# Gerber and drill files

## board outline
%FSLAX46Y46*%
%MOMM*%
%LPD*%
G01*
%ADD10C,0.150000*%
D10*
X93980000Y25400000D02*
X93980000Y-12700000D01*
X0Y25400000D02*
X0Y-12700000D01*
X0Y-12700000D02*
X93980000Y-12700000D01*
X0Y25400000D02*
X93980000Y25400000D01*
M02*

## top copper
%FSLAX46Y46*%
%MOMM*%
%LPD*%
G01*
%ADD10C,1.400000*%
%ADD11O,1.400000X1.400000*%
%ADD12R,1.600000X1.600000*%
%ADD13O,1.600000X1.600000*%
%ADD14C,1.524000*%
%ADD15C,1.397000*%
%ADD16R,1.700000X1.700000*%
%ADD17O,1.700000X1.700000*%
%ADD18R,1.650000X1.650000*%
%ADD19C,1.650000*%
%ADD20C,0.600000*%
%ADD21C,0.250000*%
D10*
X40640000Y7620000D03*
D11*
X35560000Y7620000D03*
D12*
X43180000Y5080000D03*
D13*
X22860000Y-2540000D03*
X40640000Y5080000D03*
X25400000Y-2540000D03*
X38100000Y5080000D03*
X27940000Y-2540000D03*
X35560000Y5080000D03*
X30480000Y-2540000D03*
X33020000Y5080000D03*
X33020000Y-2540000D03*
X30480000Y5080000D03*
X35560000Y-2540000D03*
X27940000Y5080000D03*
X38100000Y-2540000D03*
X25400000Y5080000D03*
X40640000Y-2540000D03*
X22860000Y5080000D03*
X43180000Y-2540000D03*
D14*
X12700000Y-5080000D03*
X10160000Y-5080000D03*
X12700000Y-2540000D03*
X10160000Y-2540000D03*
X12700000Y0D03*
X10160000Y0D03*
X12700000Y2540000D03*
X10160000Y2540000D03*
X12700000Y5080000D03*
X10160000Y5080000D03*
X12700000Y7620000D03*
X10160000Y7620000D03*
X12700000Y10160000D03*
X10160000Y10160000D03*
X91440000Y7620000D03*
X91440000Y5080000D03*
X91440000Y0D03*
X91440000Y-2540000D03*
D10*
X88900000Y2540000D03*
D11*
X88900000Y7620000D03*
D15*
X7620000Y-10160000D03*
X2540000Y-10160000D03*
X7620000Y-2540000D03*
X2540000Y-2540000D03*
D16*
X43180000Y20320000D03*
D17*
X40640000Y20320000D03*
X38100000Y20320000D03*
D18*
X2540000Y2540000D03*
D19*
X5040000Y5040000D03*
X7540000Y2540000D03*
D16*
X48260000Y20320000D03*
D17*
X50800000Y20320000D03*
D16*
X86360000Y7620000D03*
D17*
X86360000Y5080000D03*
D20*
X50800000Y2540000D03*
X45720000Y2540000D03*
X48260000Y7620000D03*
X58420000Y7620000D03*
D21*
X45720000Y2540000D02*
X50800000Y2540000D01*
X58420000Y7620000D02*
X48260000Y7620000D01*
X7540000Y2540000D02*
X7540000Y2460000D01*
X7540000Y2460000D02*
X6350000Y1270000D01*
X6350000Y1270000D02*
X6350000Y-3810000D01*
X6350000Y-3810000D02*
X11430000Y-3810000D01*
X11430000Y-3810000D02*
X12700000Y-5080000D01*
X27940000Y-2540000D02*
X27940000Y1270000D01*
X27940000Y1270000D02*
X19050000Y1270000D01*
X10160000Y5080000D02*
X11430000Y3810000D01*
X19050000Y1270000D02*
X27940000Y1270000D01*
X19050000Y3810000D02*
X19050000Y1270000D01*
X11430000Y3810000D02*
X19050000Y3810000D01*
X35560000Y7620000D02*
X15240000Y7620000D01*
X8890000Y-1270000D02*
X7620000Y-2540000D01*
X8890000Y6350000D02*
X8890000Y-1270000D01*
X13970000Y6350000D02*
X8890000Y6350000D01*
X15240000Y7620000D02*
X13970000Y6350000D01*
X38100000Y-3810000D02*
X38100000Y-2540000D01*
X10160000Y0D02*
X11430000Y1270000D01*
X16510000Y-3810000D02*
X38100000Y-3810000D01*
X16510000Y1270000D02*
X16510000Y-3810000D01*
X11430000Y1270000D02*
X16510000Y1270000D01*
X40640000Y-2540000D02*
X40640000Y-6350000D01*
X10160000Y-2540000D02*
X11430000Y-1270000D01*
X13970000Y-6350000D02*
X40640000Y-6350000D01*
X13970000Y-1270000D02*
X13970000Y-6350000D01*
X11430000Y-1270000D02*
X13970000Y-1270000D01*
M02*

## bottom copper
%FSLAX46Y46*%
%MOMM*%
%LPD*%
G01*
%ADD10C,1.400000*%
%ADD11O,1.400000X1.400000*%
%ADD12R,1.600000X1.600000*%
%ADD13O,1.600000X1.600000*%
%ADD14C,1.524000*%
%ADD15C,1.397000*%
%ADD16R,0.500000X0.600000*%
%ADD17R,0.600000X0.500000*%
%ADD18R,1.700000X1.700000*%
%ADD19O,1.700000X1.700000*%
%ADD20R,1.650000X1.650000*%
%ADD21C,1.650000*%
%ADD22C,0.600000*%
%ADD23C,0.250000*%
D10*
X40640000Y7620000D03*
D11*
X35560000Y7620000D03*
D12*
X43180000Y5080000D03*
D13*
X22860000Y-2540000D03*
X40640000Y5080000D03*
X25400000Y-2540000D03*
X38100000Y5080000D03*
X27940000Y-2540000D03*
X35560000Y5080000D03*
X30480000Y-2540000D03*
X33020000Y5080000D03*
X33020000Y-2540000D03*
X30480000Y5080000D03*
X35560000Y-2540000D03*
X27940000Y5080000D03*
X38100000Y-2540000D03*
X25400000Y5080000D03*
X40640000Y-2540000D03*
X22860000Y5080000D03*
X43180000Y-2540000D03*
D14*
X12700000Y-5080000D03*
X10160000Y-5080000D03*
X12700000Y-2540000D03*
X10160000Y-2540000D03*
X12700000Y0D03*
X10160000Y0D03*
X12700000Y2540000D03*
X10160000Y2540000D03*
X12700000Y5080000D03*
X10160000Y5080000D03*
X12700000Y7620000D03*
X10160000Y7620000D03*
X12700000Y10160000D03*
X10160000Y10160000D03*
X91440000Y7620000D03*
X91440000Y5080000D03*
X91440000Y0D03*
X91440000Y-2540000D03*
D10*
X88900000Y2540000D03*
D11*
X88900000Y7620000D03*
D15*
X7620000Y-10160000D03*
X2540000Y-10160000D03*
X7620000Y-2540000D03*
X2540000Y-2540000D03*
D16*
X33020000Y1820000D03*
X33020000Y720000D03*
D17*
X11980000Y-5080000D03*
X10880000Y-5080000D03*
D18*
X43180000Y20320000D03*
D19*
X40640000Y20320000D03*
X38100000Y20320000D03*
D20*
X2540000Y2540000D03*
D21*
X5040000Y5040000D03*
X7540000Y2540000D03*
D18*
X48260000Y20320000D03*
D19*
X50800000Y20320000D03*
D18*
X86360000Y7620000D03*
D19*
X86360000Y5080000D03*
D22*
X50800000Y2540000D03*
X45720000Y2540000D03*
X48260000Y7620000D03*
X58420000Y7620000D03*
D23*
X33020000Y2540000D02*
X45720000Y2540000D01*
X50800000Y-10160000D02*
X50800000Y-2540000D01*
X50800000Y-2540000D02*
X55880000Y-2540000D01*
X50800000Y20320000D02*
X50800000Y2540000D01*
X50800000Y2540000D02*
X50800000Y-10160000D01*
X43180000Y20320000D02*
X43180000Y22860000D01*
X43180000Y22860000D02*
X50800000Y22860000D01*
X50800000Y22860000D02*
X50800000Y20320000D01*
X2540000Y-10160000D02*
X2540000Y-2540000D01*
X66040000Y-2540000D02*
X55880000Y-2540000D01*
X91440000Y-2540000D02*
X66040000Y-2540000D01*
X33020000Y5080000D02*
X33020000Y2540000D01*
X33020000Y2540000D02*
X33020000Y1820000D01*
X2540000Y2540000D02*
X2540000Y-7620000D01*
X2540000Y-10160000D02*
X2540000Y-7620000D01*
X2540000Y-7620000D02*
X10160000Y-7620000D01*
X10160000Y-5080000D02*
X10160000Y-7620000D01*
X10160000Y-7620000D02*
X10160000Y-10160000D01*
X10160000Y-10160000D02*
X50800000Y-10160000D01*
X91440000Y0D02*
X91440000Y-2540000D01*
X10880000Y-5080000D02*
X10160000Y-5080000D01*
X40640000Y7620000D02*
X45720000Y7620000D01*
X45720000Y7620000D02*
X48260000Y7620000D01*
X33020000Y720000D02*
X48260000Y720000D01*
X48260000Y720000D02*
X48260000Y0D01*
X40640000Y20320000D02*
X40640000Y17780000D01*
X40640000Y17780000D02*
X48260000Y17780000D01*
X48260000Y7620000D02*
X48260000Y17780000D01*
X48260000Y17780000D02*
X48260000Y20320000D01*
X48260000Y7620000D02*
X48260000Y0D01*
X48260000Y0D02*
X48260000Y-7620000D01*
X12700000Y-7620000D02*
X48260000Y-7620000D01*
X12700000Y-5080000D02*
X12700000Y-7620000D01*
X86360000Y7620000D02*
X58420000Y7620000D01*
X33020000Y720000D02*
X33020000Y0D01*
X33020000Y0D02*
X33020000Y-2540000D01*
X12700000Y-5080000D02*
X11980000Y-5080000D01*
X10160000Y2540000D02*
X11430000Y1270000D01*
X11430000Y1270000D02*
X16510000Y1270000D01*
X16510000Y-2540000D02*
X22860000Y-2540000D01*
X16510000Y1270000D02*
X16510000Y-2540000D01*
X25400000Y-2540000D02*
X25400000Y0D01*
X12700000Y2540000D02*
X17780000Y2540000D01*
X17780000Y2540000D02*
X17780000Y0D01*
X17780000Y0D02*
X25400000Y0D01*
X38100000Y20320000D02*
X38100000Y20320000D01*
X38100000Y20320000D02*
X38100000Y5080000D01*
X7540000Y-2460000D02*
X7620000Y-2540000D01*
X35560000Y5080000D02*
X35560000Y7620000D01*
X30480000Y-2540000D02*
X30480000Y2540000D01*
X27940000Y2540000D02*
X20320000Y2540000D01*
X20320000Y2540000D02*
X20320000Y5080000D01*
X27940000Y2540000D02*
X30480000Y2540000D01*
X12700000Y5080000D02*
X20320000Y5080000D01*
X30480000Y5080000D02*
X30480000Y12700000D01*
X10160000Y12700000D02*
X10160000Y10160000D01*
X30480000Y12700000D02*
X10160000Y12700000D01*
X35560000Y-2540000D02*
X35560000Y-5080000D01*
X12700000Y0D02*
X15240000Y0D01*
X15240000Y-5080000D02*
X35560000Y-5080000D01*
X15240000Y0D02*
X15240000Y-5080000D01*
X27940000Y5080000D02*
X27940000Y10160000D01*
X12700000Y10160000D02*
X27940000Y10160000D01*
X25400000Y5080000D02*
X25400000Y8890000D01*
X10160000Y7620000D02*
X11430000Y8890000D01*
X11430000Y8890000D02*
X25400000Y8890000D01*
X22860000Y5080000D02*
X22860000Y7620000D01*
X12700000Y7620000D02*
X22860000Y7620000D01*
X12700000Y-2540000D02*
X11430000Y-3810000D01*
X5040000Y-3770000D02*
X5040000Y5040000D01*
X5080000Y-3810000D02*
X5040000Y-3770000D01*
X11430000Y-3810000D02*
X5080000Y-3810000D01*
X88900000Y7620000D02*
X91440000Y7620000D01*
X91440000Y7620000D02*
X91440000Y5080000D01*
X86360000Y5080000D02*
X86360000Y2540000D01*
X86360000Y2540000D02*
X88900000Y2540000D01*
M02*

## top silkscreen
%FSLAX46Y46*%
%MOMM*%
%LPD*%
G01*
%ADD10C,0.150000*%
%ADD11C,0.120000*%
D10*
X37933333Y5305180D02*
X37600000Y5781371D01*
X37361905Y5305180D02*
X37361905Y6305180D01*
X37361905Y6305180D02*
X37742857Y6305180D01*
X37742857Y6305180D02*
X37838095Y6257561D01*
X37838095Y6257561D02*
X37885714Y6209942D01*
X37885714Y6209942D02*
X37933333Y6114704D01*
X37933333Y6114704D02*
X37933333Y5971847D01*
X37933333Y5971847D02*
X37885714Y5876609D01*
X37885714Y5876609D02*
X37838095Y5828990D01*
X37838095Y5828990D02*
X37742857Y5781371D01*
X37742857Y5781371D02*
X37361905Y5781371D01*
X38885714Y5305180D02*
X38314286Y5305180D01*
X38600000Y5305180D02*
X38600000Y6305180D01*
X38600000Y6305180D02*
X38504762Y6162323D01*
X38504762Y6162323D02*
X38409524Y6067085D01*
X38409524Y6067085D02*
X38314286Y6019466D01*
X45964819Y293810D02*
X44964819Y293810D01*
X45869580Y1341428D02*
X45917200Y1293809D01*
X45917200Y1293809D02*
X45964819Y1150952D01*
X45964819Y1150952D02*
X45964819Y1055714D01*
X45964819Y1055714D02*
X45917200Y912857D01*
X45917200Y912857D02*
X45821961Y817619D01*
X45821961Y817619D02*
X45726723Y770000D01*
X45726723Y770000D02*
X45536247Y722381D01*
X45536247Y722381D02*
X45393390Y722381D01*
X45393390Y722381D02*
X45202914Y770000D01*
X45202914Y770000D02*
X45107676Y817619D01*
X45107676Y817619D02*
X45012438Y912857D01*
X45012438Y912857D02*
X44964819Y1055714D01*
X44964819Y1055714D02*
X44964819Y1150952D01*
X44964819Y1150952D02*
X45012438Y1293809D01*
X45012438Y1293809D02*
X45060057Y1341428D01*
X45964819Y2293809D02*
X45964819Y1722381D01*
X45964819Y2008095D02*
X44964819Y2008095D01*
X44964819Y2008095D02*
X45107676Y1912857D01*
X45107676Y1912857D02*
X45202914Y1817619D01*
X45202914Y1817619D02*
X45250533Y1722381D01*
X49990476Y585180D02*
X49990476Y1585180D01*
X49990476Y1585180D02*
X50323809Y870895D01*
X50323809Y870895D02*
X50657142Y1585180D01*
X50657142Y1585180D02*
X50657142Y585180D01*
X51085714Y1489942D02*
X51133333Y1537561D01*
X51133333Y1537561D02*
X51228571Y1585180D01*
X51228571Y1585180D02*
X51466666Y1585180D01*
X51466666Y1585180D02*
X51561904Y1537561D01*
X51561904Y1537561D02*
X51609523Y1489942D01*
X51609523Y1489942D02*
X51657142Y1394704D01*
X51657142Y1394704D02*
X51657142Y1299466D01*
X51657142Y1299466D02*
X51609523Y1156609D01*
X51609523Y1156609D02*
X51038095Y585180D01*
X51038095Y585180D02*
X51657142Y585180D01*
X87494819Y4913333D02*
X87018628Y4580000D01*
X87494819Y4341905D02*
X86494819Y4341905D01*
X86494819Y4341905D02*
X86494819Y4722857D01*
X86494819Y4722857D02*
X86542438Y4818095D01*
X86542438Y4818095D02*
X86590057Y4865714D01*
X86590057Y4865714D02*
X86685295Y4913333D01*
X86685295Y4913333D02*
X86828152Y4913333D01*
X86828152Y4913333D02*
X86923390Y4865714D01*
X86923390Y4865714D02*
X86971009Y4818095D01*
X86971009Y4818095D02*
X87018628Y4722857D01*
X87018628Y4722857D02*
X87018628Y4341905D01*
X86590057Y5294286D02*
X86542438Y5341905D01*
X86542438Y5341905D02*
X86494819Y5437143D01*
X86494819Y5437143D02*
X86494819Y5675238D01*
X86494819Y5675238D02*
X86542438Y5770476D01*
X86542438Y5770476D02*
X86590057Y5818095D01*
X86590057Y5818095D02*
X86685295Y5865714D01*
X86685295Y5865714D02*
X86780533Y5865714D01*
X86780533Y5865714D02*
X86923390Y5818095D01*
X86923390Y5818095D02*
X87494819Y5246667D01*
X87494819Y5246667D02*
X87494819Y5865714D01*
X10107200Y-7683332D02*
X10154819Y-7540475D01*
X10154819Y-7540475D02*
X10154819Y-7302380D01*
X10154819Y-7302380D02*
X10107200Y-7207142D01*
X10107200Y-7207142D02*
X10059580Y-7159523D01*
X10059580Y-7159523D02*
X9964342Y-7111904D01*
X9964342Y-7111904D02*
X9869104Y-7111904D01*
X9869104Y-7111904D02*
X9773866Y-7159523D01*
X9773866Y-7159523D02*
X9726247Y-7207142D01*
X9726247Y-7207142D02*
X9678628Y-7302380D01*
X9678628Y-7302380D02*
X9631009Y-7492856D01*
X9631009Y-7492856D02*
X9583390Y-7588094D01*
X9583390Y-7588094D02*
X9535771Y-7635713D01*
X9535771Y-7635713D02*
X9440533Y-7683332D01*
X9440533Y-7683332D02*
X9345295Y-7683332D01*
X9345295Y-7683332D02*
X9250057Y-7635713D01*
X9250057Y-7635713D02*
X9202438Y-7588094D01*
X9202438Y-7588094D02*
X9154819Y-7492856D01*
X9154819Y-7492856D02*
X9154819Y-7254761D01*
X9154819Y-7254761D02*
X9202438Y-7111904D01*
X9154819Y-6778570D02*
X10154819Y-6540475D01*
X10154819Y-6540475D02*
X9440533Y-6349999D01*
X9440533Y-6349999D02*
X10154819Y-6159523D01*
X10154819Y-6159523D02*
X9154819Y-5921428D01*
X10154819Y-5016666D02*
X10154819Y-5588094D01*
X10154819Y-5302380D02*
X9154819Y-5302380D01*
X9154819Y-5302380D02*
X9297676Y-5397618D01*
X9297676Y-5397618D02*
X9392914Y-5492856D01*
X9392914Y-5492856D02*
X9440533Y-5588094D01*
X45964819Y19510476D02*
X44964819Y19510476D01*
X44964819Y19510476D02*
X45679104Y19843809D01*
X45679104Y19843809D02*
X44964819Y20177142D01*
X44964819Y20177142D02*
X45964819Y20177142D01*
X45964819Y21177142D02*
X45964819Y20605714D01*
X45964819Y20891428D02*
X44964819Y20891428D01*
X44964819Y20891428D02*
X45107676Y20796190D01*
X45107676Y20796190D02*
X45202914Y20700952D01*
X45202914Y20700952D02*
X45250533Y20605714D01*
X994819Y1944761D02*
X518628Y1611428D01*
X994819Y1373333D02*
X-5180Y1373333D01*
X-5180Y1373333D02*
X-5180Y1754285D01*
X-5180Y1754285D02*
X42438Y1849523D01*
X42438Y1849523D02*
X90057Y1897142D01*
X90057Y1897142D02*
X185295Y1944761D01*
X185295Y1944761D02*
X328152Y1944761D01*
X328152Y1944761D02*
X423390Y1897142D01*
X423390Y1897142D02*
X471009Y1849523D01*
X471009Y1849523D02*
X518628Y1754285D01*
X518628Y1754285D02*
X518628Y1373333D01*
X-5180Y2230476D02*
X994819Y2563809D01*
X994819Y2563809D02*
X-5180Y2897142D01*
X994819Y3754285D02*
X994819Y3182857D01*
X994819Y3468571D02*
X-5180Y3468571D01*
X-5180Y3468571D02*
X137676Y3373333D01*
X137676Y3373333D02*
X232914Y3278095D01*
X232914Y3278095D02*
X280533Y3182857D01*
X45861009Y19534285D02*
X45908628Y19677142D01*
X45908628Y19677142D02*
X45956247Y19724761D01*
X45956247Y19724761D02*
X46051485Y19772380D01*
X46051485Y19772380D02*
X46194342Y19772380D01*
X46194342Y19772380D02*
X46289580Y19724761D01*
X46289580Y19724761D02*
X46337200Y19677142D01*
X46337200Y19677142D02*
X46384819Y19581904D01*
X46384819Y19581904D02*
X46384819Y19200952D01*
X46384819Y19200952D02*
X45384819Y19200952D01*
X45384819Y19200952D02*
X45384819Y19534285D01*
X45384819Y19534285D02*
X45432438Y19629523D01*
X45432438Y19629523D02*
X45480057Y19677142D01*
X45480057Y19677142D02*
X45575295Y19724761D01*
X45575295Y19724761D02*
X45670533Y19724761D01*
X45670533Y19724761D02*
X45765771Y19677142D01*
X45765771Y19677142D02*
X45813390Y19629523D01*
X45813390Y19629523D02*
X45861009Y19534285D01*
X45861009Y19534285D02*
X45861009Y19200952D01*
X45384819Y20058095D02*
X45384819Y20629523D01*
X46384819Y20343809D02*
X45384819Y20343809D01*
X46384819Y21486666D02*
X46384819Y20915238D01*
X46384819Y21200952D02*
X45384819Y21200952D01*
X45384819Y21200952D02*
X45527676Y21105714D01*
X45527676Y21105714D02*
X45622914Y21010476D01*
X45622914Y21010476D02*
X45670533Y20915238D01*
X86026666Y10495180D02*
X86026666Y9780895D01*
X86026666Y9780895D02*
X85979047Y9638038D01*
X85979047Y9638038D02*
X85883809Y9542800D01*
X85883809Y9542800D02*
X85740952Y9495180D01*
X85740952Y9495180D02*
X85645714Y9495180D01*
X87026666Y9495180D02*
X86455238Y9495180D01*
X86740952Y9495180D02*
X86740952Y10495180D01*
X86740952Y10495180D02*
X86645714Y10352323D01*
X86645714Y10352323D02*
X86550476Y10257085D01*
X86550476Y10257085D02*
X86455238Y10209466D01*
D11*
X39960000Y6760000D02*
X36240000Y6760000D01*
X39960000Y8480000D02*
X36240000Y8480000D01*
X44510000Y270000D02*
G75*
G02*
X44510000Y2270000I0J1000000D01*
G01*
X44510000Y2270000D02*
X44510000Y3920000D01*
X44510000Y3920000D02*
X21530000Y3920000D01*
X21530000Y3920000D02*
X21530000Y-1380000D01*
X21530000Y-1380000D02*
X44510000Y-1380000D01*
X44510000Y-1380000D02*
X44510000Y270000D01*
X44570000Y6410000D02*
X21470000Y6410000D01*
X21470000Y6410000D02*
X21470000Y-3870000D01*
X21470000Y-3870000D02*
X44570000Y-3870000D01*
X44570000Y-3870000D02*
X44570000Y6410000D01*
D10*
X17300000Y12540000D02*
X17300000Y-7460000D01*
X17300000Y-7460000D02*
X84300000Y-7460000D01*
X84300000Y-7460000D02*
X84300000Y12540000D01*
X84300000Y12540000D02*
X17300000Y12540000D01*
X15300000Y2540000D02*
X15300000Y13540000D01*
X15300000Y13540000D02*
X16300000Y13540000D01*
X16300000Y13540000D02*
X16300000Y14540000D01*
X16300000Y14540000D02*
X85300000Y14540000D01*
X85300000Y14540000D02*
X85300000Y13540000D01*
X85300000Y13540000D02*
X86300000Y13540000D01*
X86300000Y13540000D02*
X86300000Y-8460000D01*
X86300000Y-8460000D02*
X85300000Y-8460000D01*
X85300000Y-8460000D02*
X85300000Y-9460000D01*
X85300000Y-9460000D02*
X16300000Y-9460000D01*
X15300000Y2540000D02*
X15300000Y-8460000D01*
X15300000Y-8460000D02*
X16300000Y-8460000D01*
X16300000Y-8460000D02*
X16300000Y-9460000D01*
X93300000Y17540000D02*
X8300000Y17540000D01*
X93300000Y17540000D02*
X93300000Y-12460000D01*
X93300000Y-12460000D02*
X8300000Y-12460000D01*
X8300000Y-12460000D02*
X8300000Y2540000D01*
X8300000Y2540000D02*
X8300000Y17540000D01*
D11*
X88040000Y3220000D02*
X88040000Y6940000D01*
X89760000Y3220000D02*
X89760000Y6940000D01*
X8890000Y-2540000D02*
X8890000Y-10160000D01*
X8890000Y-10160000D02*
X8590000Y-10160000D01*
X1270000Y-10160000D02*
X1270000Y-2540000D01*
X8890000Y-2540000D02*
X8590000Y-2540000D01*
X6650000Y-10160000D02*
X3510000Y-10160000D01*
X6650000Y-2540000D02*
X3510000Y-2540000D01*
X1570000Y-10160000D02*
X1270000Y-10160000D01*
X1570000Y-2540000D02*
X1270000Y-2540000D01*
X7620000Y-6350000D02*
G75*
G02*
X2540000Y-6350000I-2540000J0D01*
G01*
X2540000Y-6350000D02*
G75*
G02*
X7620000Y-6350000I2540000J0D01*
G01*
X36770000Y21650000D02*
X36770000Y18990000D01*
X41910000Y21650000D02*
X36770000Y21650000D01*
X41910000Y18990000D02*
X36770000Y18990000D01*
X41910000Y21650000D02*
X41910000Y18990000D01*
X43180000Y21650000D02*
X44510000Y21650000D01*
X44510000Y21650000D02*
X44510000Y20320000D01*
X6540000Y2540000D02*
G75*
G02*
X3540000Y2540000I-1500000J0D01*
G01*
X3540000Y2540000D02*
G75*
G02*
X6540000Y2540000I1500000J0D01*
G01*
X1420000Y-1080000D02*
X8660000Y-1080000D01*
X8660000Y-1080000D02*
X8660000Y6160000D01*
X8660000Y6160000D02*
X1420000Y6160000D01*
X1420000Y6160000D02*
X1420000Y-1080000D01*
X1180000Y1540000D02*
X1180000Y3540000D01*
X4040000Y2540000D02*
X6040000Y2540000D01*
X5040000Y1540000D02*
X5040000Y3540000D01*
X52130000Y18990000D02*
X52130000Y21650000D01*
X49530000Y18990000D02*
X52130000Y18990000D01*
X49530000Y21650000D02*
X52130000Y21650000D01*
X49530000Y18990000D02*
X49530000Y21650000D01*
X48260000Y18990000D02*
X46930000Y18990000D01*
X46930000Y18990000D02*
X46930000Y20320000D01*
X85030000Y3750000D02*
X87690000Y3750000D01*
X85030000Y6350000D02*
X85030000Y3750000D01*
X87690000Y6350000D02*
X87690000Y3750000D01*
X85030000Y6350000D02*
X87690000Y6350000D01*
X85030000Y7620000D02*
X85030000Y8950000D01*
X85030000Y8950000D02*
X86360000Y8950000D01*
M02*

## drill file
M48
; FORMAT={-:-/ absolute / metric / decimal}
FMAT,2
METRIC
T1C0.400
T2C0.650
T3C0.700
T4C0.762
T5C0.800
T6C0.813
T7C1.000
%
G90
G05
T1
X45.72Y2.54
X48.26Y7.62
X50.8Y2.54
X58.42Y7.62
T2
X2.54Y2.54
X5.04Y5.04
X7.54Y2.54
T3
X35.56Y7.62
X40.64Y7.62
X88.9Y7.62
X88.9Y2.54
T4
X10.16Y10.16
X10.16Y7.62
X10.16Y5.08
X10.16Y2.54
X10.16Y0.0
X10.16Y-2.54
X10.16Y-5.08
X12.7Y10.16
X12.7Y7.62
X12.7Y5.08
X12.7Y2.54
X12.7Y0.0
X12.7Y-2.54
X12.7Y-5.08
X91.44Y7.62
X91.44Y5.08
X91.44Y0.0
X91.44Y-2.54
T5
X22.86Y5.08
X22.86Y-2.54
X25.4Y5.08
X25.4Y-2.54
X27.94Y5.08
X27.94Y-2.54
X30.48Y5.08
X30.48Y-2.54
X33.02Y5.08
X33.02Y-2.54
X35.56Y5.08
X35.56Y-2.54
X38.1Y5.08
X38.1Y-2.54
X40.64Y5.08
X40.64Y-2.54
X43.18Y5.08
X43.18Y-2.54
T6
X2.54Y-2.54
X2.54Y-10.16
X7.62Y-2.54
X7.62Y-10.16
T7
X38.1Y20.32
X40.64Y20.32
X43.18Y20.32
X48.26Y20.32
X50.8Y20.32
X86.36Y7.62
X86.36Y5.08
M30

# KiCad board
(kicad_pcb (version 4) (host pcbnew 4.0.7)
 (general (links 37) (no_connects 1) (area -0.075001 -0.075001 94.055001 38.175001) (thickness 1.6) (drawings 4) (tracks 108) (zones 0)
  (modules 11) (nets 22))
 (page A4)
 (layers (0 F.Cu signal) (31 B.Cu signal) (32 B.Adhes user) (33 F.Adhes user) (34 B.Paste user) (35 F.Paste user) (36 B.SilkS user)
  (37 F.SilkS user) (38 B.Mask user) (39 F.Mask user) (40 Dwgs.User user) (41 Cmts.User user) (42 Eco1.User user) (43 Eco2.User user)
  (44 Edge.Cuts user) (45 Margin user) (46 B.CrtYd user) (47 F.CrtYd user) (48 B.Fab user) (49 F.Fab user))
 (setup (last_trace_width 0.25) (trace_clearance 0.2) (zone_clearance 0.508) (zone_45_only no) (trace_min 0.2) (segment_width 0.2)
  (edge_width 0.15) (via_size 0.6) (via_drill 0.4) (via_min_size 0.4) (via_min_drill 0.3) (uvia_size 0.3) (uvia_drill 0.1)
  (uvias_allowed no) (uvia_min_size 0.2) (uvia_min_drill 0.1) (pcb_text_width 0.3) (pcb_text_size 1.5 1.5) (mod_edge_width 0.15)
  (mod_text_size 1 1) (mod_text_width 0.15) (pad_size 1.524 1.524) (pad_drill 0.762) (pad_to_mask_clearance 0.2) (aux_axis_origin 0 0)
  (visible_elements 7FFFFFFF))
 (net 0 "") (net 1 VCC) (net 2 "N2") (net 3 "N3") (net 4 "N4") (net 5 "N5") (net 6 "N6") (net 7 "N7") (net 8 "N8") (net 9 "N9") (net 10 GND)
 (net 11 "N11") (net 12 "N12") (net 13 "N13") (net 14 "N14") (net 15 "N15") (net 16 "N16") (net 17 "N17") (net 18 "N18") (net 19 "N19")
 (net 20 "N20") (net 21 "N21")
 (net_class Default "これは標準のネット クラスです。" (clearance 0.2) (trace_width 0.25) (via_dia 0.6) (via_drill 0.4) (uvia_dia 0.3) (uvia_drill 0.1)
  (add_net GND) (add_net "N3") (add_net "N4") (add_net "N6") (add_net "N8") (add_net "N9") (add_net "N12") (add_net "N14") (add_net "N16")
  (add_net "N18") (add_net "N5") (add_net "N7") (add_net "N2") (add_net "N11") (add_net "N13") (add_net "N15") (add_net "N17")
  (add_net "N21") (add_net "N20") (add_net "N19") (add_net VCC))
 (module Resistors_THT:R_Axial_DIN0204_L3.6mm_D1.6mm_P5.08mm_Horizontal (layer F.Cu) (at 40.64 -7.62 180)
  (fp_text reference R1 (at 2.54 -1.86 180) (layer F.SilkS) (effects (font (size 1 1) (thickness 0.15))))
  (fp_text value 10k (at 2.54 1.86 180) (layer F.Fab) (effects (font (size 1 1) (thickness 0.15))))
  (fp_line (start 0.68 -0.86) (end 4.4 -0.86) (layer F.SilkS) (width 0.12))
  (fp_line (start 0.68 0.86) (end 4.4 0.86) (layer F.SilkS) (width 0.12))
  (pad 1 thru_hole circle (at 0 0 180) (size 1.4 1.4) (drill 0.7) (layers *.Cu *.Mask) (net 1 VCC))
  (pad 2 thru_hole oval (at 5.08 0 180) (size 1.4 1.4) (drill 0.7) (layers *.Cu *.Mask) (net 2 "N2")))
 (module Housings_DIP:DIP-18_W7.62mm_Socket (layer F.Cu) (at 43.18 -5.08 270)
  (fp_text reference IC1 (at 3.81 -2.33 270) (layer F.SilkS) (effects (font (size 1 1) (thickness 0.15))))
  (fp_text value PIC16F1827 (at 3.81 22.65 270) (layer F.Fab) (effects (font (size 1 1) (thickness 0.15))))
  (fp_arc (start 3.81 -1.33) (end 2.81 -1.33) (angle -180) (layer F.SilkS) (width 0.12))
  (fp_line (start 2.81 -1.33) (end 1.16 -1.33) (layer F.SilkS) (width 0.12))
  (fp_line (start 1.16 -1.33) (end 1.16 21.65) (layer F.SilkS) (width 0.12))
  (fp_line (start 1.16 21.65) (end 6.46 21.65) (layer F.SilkS) (width 0.12))
  (fp_line (start 6.46 21.65) (end 6.46 -1.33) (layer F.SilkS) (width 0.12))
  (fp_line (start 6.46 -1.33) (end 4.81 -1.33) (layer F.SilkS) (width 0.12))
  (fp_line (start -1.33 -1.39) (end -1.33 21.71) (layer F.SilkS) (width 0.12))
  (fp_line (start -1.33 21.71) (end 8.95 21.71) (layer F.SilkS) (width 0.12))
  (fp_line (start 8.95 21.71) (end 8.95 -1.39) (layer F.SilkS) (width 0.12))
  (fp_line (start 8.95 -1.39) (end -1.33 -1.39) (layer F.SilkS) (width 0.12))
  (pad 1 thru_hole rect (at 0 0 270) (size 1.6 1.6) (drill 0.8) (layers *.Cu *.Mask) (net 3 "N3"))
  (pad 10 thru_hole oval (at 7.62 20.32 270) (size 1.6 1.6) (drill 0.8) (layers *.Cu *.Mask) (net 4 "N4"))
  (pad 2 thru_hole oval (at 0 2.54 270) (size 1.6 1.6) (drill 0.8) (layers *.Cu *.Mask) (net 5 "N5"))
  (pad 11 thru_hole oval (at 7.62 17.78 270) (size 1.6 1.6) (drill 0.8) (layers *.Cu *.Mask) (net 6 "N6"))
  (pad 3 thru_hole oval (at 0 5.08 270) (size 1.6 1.6) (drill 0.8) (layers *.Cu *.Mask) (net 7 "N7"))
  (pad 12 thru_hole oval (at 7.62 15.24 270) (size 1.6 1.6) (drill 0.8) (layers *.Cu *.Mask) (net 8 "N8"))
  (pad 4 thru_hole oval (at 0 7.62 270) (size 1.6 1.6) (drill 0.8) (layers *.Cu *.Mask) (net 2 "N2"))
  (pad 13 thru_hole oval (at 7.62 12.7 270) (size 1.6 1.6) (drill 0.8) (layers *.Cu *.Mask) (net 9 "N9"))
  (pad 5 thru_hole oval (at 0 10.16 270) (size 1.6 1.6) (drill 0.8) (layers *.Cu *.Mask) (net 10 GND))
  (pad 14 thru_hole oval (at 7.62 10.16 270) (size 1.6 1.6) (drill 0.8) (layers *.Cu *.Mask) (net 1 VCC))
  (pad 6 thru_hole oval (at 0 12.7 270) (size 1.6 1.6) (drill 0.8) (layers *.Cu *.Mask) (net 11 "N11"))
  (pad 15 thru_hole oval (at 7.62 7.62 270) (size 1.6 1.6) (drill 0.8) (layers *.Cu *.Mask) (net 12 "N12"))
  (pad 7 thru_hole oval (at 0 15.24 270) (size 1.6 1.6) (drill 0.8) (layers *.Cu *.Mask) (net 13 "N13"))
  (pad 16 thru_hole oval (at 7.62 5.08 270) (size 1.6 1.6) (drill 0.8) (layers *.Cu *.Mask) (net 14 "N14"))
  (pad 8 thru_hole oval (at 0 17.78 270) (size 1.6 1.6) (drill 0.8) (layers *.Cu *.Mask) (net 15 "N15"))
  (pad 17 thru_hole oval (at 7.62 2.54 270) (size 1.6 1.6) (drill 0.8) (layers *.Cu *.Mask) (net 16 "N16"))
  (pad 9 thru_hole oval (at 0 20.32 270) (size 1.6 1.6) (drill 0.8) (layers *.Cu *.Mask) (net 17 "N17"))
  (pad 18 thru_hole oval (at 7.62 0 270) (size 1.6 1.6) (drill 0.8) (layers *.Cu *.Mask) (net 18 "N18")))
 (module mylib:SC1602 (layer F.Cu) (at 50.8 -2.54)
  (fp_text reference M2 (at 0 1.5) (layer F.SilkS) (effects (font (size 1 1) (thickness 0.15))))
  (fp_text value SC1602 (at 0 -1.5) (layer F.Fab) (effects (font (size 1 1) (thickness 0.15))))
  (fp_line (start -33.5 -10) (end -33.5 10) (layer F.SilkS) (width 0.15))
  (fp_line (start -33.5 10) (end 33.5 10) (layer F.SilkS) (width 0.15))
  (fp_line (start 33.5 10) (end 33.5 -10) (layer F.SilkS) (width 0.15))
  (fp_line (start 33.5 -10) (end -33.5 -10) (layer F.SilkS) (width 0.15))
  (fp_line (start -35.5 0) (end -35.5 -11) (layer F.SilkS) (width 0.15))
  (fp_line (start -35.5 -11) (end -34.5 -11) (layer F.SilkS) (width 0.15))
  (fp_line (start -34.5 -11) (end -34.5 -12) (layer F.SilkS) (width 0.15))
  (fp_line (start -34.5 -12) (end 34.5 -12) (layer F.SilkS) (width 0.15))
  (fp_line (start 34.5 -12) (end 34.5 -11) (layer F.SilkS) (width 0.15))
  (fp_line (start 34.5 -11) (end 35.5 -11) (layer F.SilkS) (width 0.15))
  (fp_line (start 35.5 -11) (end 35.5 11) (layer F.SilkS) (width 0.15))
  (fp_line (start 35.5 11) (end 34.5 11) (layer F.SilkS) (width 0.15))
  (fp_line (start 34.5 11) (end 34.5 12) (layer F.SilkS) (width 0.15))
  (fp_line (start 34.5 12) (end -34.5 12) (layer F.SilkS) (width 0.15))
  (fp_line (start -35.5 0) (end -35.5 11) (layer F.SilkS) (width 0.15))
  (fp_line (start -35.5 11) (end -34.5 11) (layer F.SilkS) (width 0.15))
  (fp_line (start -34.5 11) (end -34.5 12) (layer F.SilkS) (width 0.15))
  (fp_line (start 42.5 -15) (end -42.5 -15) (layer F.SilkS) (width 0.15))
  (fp_line (start 42.5 -15) (end 42.5 15) (layer F.SilkS) (width 0.15))
  (fp_line (start 42.5 15) (end -42.5 15) (layer F.SilkS) (width 0.15))
  (fp_line (start -42.5 15) (end -42.5 0) (layer F.SilkS) (width 0.15))
  (fp_line (start -42.5 0) (end -42.5 -15) (layer F.SilkS) (width 0.15))
  (pad 1 thru_hole circle (at -38.1 7.62) (size 1.524 1.524) (drill 0.762) (layers *.Cu *.Mask) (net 1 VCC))
  (pad 2 thru_hole circle (at -40.64 7.62) (size 1.524 1.524) (drill 0.762) (layers *.Cu *.Mask) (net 10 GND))
  (pad 3 thru_hole circle (at -38.1 5.08) (size 1.524 1.524) (drill 0.762) (layers *.Cu *.Mask) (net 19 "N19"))
  (pad 4 thru_hole circle (at -40.64 5.08) (size 1.524 1.524) (drill 0.762) (layers *.Cu *.Mask) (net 16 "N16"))
  (pad 5 thru_hole circle (at -38.1 2.54) (size 1.524 1.524) (drill 0.762) (layers *.Cu *.Mask) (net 12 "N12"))
  (pad 6 thru_hole circle (at -40.64 2.54) (size 1.524 1.524) (drill 0.762) (layers *.Cu *.Mask) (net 14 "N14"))
  (pad 7 thru_hole circle (at -38.1 0) (size 1.524 1.524) (drill 0.762) (layers *.Cu *.Mask) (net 6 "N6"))
  (pad 8 thru_hole circle (at -40.64 0) (size 1.524 1.524) (drill 0.762) (layers *.Cu *.Mask) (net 4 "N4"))
  (pad 9 thru_hole circle (at -38.1 -2.54) (size 1.524 1.524) (drill 0.762) (layers *.Cu *.Mask) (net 9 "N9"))
  (pad 10 thru_hole circle (at -40.64 -2.54) (size 1.524 1.524) (drill 0.762) (layers *.Cu *.Mask) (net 8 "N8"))
  (pad 11 thru_hole circle (at -38.1 -5.08) (size 1.524 1.524) (drill 0.762) (layers *.Cu *.Mask) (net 17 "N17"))
  (pad 12 thru_hole circle (at -40.64 -5.08) (size 1.524 1.524) (drill 0.762) (layers *.Cu *.Mask) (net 15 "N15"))
  (pad 13 thru_hole circle (at -38.1 -7.62) (size 1.524 1.524) (drill 0.762) (layers *.Cu *.Mask) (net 13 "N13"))
  (pad 14 thru_hole circle (at -40.64 -7.62) (size 1.524 1.524) (drill 0.762) (layers *.Cu *.Mask) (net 11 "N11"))
  (pad 15 thru_hole circle (at 40.64 -5.08) (size 1.524 1.524) (drill 0.762) (layers *.Cu *.Mask) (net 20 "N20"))
  (pad 15 thru_hole circle (at 40.64 -2.54) (size 1.524 1.524) (drill 0.762) (layers *.Cu *.Mask) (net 20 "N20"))
  (pad 16 thru_hole circle (at 40.64 2.54) (size 1.524 1.524) (drill 0.762) (layers *.Cu *.Mask) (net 10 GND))
  (pad 16 thru_hole circle (at 40.64 5.08) (size 1.524 1.524) (drill 0.762) (layers *.Cu *.Mask) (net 10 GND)))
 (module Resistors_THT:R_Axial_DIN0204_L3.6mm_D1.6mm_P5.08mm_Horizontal (layer F.Cu) (at 88.9 -2.54 90)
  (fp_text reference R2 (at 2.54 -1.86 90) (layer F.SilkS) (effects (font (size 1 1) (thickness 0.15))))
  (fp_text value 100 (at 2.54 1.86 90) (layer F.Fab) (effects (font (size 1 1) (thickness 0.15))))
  (fp_line (start 0.68 -0.86) (end 4.4 -0.86) (layer F.SilkS) (width 0.12))
  (fp_line (start 0.68 0.86) (end 4.4 0.86) (layer F.SilkS) (width 0.12))
  (pad 1 thru_hole circle (at 0 0 90) (size 1.4 1.4) (drill 0.7) (layers *.Cu *.Mask) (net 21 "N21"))
  (pad 2 thru_hole oval (at 5.08 0 90) (size 1.4 1.4) (drill 0.7) (layers *.Cu *.Mask) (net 20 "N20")))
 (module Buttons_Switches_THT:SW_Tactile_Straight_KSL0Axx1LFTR (layer F.Cu) (at 7.62 2.54 270)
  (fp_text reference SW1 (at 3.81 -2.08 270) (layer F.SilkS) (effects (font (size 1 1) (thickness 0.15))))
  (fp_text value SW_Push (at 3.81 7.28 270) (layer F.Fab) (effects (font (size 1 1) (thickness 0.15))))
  (fp_line (start 0 -1.27) (end 7.62 -1.27) (layer F.SilkS) (width 0.12))
  (fp_line (start 7.62 -1.27) (end 7.62 -0.97) (layer F.SilkS) (width 0.12))
  (fp_line (start 7.62 6.35) (end 0 6.35) (layer F.SilkS) (width 0.12))
  (fp_line (start 0 -1.27) (end 0 -0.97) (layer F.SilkS) (width 0.12))
  (fp_line (start 7.62 0.97) (end 7.62 4.11) (layer F.SilkS) (width 0.12))
  (fp_line (start 0 0.97) (end 0 4.11) (layer F.SilkS) (width 0.12))
  (fp_line (start 7.62 6.05) (end 7.62 6.35) (layer F.SilkS) (width 0.12))
  (fp_line (start 0 6.05) (end 0 6.35) (layer F.SilkS) (width 0.12))
  (fp_circle (center 3.81 2.54) (end 3.81 0) (layer F.SilkS) (width 0.12))
  (pad 1 thru_hole circle (at 7.62 0 270) (size 1.397 1.397) (drill 0.8128) (layers *.Cu *.Mask) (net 2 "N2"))
  (pad 2 thru_hole circle (at 7.62 5.08 270) (size 1.397 1.397) (drill 0.8128) (layers *.Cu *.Mask) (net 10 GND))
  (pad 1 thru_hole circle (at 0 0 270) (size 1.397 1.397) (drill 0.8128) (layers *.Cu *.Mask) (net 2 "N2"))
  (pad 2 thru_hole circle (at 0 5.08 270) (size 1.397 1.397) (drill 0.8128) (layers *.Cu *.Mask) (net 10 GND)))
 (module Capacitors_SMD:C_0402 (layer B.Cu) (at 33.02 -1.27 270)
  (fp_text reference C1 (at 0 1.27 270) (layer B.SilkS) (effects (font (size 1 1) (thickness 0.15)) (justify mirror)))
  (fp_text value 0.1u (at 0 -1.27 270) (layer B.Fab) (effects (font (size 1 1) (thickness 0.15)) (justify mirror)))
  (pad 1 smd rect (at -0.55 0 270) (size 0.6 0.5) (layers B.Cu B.Paste B.Mask) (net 10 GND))
  (pad 2 smd rect (at 0.55 0 270) (size 0.6 0.5) (layers B.Cu B.Paste B.Mask) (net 1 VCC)))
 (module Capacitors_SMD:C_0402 (layer B.Cu) (at 11.43 5.08 180)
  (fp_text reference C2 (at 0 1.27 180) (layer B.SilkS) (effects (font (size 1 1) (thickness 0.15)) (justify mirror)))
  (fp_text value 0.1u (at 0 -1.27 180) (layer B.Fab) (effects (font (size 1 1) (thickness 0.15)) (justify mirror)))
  (pad 1 smd rect (at -0.55 0 180) (size 0.6 0.5) (layers B.Cu B.Paste B.Mask) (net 1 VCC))
  (pad 2 smd rect (at 0.55 0 180) (size 0.6 0.5) (layers B.Cu B.Paste B.Mask) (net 10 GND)))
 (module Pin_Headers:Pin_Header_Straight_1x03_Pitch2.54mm (layer F.Cu) (at 43.18 -20.32 270)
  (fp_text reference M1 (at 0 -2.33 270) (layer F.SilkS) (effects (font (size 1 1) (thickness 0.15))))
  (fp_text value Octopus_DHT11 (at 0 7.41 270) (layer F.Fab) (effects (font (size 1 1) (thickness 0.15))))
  (fp_line (start -1.33 6.41) (end 1.33 6.41) (layer F.SilkS) (width 0.12))
  (fp_line (start -1.33 1.27) (end -1.33 6.41) (layer F.SilkS) (width 0.12))
  (fp_line (start 1.33 1.27) (end 1.33 6.41) (layer F.SilkS) (width 0.12))
  (fp_line (start -1.33 1.27) (end 1.33 1.27) (layer F.SilkS) (width 0.12))
  (fp_line (start -1.33 0) (end -1.33 -1.33) (layer F.SilkS) (width 0.12))
  (fp_line (start -1.33 -1.33) (end 0 -1.33) (layer F.SilkS) (width 0.12))
  (pad 1 thru_hole rect (at 0 0 270) (size 1.7 1.7) (drill 1) (layers *.Cu *.Mask) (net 10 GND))
  (pad 2 thru_hole oval (at 0 2.54 270) (size 1.7 1.7) (drill 1) (layers *.Cu *.Mask) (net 1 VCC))
  (pad 3 thru_hole oval (at 0 5.08 270) (size 1.7 1.7) (drill 1) (layers *.Cu *.Mask) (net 7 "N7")))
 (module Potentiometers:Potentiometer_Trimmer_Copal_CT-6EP (layer F.Cu) (at 2.54 -2.54 90)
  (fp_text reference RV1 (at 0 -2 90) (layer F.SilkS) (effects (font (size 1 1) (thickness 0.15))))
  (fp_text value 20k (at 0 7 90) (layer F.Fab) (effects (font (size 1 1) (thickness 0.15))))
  (fp_circle (center 0 2.5) (end 1.5 2.5) (layer F.SilkS) (width 0.12))
  (fp_line (start -3.62 -1.12) (end -3.62 6.12) (layer F.SilkS) (width 0.12))
  (fp_line (start -3.62 6.12) (end 3.62 6.12) (layer F.SilkS) (width 0.12))
  (fp_line (start 3.62 6.12) (end 3.62 -1.12) (layer F.SilkS) (width 0.12))
  (fp_line (start 3.62 -1.12) (end -3.62 -1.12) (layer F.SilkS) (width 0.12))
  (fp_line (start -1 -1.36) (end 1 -1.36) (layer F.SilkS) (width 0.12))
  (fp_line (start 0 1.5) (end 0 3.5) (layer F.SilkS) (width 0.12))
  (fp_line (start -1 2.5) (end 1 2.5) (layer F.SilkS) (width 0.12))
  (pad 1 thru_hole rect (at 0 0 90) (size 1.65 1.65) (drill 0.65) (layers *.Cu *.Mask) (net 10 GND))
  (pad 2 thru_hole circle (at 2.5 2.5 90) (size 1.65 1.65) (drill 0.65) (layers *.Cu *.Mask) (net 19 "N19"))
  (pad 3 thru_hole circle (at 0 5 90) (size 1.65 1.65) (drill 0.65) (layers *.Cu *.Mask) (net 1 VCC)))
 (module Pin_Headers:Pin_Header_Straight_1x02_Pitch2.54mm (layer F.Cu) (at 48.26 -20.32 90)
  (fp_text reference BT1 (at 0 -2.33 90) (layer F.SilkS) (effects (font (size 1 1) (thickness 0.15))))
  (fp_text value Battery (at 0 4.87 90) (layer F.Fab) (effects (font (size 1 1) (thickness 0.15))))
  (fp_line (start -1.33 3.87) (end 1.33 3.87) (layer F.SilkS) (width 0.12))
  (fp_line (start -1.33 1.27) (end -1.33 3.87) (layer F.SilkS) (width 0.12))
  (fp_line (start 1.33 1.27) (end 1.33 3.87) (layer F.SilkS) (width 0.12))
  (fp_line (start -1.33 1.27) (end 1.33 1.27) (layer F.SilkS) (width 0.12))
  (fp_line (start -1.33 0) (end -1.33 -1.33) (layer F.SilkS) (width 0.12))
  (fp_line (start -1.33 -1.33) (end 0 -1.33) (layer F.SilkS) (width 0.12))
  (pad 1 thru_hole rect (at 0 0 90) (size 1.7 1.7) (drill 1) (layers *.Cu *.Mask) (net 1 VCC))
  (pad 2 thru_hole oval (at 0 2.54 90) (size 1.7 1.7) (drill 1) (layers *.Cu *.Mask) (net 10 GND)))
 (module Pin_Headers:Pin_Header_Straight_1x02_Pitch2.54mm (layer F.Cu) (at 86.36 -7.62)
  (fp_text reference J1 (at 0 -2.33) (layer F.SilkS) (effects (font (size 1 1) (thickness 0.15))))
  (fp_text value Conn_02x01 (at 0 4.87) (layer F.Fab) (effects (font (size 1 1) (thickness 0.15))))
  (fp_line (start -1.33 3.87) (end 1.33 3.87) (layer F.SilkS) (width 0.12))
  (fp_line (start -1.33 1.27) (end -1.33 3.87) (layer F.SilkS) (width 0.12))
  (fp_line (start 1.33 1.27) (end 1.33 3.87) (layer F.SilkS) (width 0.12))
  (fp_line (start -1.33 1.27) (end 1.33 1.27) (layer F.SilkS) (width 0.12))
  (fp_line (start -1.33 0) (end -1.33 -1.33) (layer F.SilkS) (width 0.12))
  (fp_line (start -1.33 -1.33) (end 0 -1.33) (layer F.SilkS) (width 0.12))
  (pad 1 thru_hole rect (at 0 0) (size 1.7 1.7) (drill 1) (layers *.Cu *.Mask) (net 1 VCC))
  (pad 2 thru_hole oval (at 0 2.54) (size 1.7 1.7) (drill 1) (layers *.Cu *.Mask) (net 21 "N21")))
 (gr_line (start 93.98 -25.4) (end 93.98 12.7) (angle 90) (layer Edge.Cuts) (width 0.15))
 (gr_line (start 0 -25.4) (end 0 12.7) (angle 90) (layer Edge.Cuts) (width 0.15))
 (gr_line (start 0 12.7) (end 93.98 12.7) (angle 90) (layer Edge.Cuts) (width 0.15))
 (gr_line (start 0 -25.4) (end 93.98 -25.4) (angle 90) (layer Edge.Cuts) (width 0.15))
 (via (at 50.8 -2.54) (size 0.6) (drill 0.4) (layers F.Cu B.Cu) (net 10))
 (segment (start 33.02 -2.54) (end 45.72 -2.54) (width 0.25) (layer B.Cu) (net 10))
 (via (at 45.72 -2.54) (size 0.6) (drill 0.4) (layers F.Cu B.Cu) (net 10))
 (segment (start 45.72 -2.54) (end 50.8 -2.54) (width 0.25) (layer F.Cu) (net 10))
 (segment (start 50.8 10.16) (end 50.8 2.54) (width 0.25) (layer B.Cu) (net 10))
 (segment (start 50.8 2.54) (end 55.88 2.54) (width 0.25) (layer B.Cu) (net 10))
 (segment (start 50.8 -20.32) (end 50.8 -2.54) (width 0.25) (layer B.Cu) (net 10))
 (segment (start 50.8 -2.54) (end 50.8 10.16) (width 0.25) (layer B.Cu) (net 10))
 (segment (start 43.18 -20.32) (end 43.18 -22.86) (width 0.25) (layer B.Cu) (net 10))
 (segment (start 43.18 -22.86) (end 50.8 -22.86) (width 0.25) (layer B.Cu) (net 10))
 (segment (start 50.8 -22.86) (end 50.8 -20.32) (width 0.25) (layer B.Cu) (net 10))
 (segment (start 2.54 10.16) (end 2.54 2.54) (width 0.25) (layer B.Cu) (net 10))
 (segment (start 66.04 2.54) (end 55.88 2.54) (width 0.25) (layer B.Cu) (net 10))
 (segment (start 91.44 2.54) (end 66.04 2.54) (width 0.25) (layer B.Cu) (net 10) (status 10))
 (segment (start 33.02 -5.08) (end 33.02 -2.54) (width 0.25) (layer B.Cu) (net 10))
 (segment (start 33.02 -2.54) (end 33.02 -1.82) (width 0.25) (layer B.Cu) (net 10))
 (segment (start 2.54 -2.54) (end 2.54 7.62) (width 0.25) (layer B.Cu) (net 10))
 (segment (start 2.54 10.16) (end 2.54 7.62) (width 0.25) (layer B.Cu) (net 10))
 (segment (start 2.54 7.62) (end 10.16 7.62) (width 0.25) (layer B.Cu) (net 10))
 (segment (start 10.16 5.08) (end 10.16 7.62) (width 0.25) (layer B.Cu) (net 10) (status 10))
 (segment (start 10.16 7.62) (end 10.16 10.16) (width 0.25) (layer B.Cu) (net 10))
 (segment (start 10.16 10.16) (end 50.8 10.16) (width 0.25) (layer B.Cu) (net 10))
 (segment (start 91.44 0) (end 91.44 2.54) (width 0.25) (layer B.Cu) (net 10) (status 30))
 (segment (start 10.88 5.08) (end 10.16 5.08) (width 0.25) (layer B.Cu) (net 10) (status 30))
 (segment (start 40.64 -7.62) (end 45.72 -7.62) (width 0.25) (layer B.Cu) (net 1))
 (segment (start 45.72 -7.62) (end 48.26 -7.62) (width 0.25) (layer B.Cu) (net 1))
 (segment (start 33.02 -0.72) (end 48.26 -0.72) (width 0.25) (layer B.Cu) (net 1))
 (segment (start 48.26 -0.72) (end 48.26 0) (width 0.25) (layer B.Cu) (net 1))
 (segment (start 40.64 -20.32) (end 40.64 -17.78) (width 0.25) (layer B.Cu) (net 1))
 (segment (start 40.64 -17.78) (end 48.26 -17.78) (width 0.25) (layer B.Cu) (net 1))
 (segment (start 48.26 -7.62) (end 48.26 -17.78) (width 0.25) (layer B.Cu) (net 1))
 (segment (start 48.26 -17.78) (end 48.26 -20.32) (width 0.25) (layer B.Cu) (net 1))
 (segment (start 48.26 -7.62) (end 48.26 0) (width 0.25) (layer B.Cu) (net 1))
 (segment (start 48.26 0) (end 48.26 7.62) (width 0.25) (layer B.Cu) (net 1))
 (segment (start 12.7 7.62) (end 48.26 7.62) (width 0.25) (layer B.Cu) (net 1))
 (segment (start 12.7 5.08) (end 12.7 7.62) (width 0.25) (layer B.Cu) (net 1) (status 10))
 (segment (start 86.36 -7.62) (end 58.42 -7.62) (width 0.25) (layer B.Cu) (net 1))
 (via (at 48.26 -7.62) (size 0.6) (drill 0.4) (layers F.Cu B.Cu) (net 1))
 (segment (start 58.42 -7.62) (end 48.26 -7.62) (width 0.25) (layer F.Cu) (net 1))
 (via (at 58.42 -7.62) (size 0.6) (drill 0.4) (layers F.Cu B.Cu) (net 1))
 (segment (start 33.02 -0.72) (end 33.02 0) (width 0.25) (layer B.Cu) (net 1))
 (segment (start 33.02 0) (end 33.02 2.54) (width 0.25) (layer B.Cu) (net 1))
 (segment (start 7.54 -2.54) (end 7.54 -2.46) (width 0.25) (layer F.Cu) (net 1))
 (segment (start 7.54 -2.46) (end 6.35 -1.27) (width 0.25) (layer F.Cu) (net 1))
 (segment (start 6.35 -1.27) (end 6.35 3.81) (width 0.25) (layer F.Cu) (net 1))
 (segment (start 6.35 3.81) (end 11.43 3.81) (width 0.25) (layer F.Cu) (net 1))
 (segment (start 11.43 3.81) (end 12.7 5.08) (width 0.25) (layer F.Cu) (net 1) (status 20))
 (segment (start 12.7 5.08) (end 11.98 5.08) (width 0.25) (layer B.Cu) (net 1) (status 30))
 (segment (start 10.16 -2.54) (end 11.43 -1.27) (width 0.25) (layer B.Cu) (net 4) (status 10))
 (segment (start 11.43 -1.27) (end 16.51 -1.27) (width 0.25) (layer B.Cu) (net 4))
 (segment (start 16.51 2.54) (end 22.86 2.54) (width 0.25) (layer B.Cu) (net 4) (status 20))
 (segment (start 16.51 -1.27) (end 16.51 2.54) (width 0.25) (layer B.Cu) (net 4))
 (segment (start 25.4 2.54) (end 25.4 0) (width 0.25) (layer B.Cu) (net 6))
 (segment (start 12.7 -2.54) (end 17.78 -2.54) (width 0.25) (layer B.Cu) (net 6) (status 10))
 (segment (start 17.78 -2.54) (end 17.78 0) (width 0.25) (layer B.Cu) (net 6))
 (segment (start 17.78 0) (end 25.4 0) (width 0.25) (layer B.Cu) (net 6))
 (segment (start 38.1 -20.32) (end 38.1 -20.32) (width 0.25) (layer B.Cu) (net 7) (status 10))
 (segment (start 38.1 -20.32) (end 38.1 -5.08) (width 0.25) (layer B.Cu) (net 7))
 (segment (start 27.94 2.54) (end 27.94 -1.27) (width 0.25) (layer F.Cu) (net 8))
 (segment (start 27.94 -1.27) (end 19.05 -1.27) (width 0.25) (layer F.Cu) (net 8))
 (segment (start 10.16 -5.08) (end 11.43 -3.81) (width 0.25) (layer F.Cu) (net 8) (status 10))
 (segment (start 19.05 -1.27) (end 27.94 -1.27) (width 0.25) (layer F.Cu) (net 8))
 (segment (start 19.05 -3.81) (end 19.05 -1.27) (width 0.25) (layer F.Cu) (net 8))
 (segment (start 11.43 -3.81) (end 19.05 -3.81) (width 0.25) (layer F.Cu) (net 8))
 (segment (start 35.56 -7.62) (end 15.24 -7.62) (width 0.25) (layer F.Cu) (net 2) (status 10))
 (segment (start 8.89 1.27) (end 7.62 2.54) (width 0.25) (layer F.Cu) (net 2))
 (segment (start 8.89 -6.35) (end 8.89 1.27) (width 0.25) (layer F.Cu) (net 2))
 (segment (start 13.97 -6.35) (end 8.89 -6.35) (width 0.25) (layer F.Cu) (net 2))
 (segment (start 15.24 -7.62) (end 13.97 -6.35) (width 0.25) (layer F.Cu) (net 2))
 (segment (start 7.54 2.46) (end 7.62 2.54) (width 0.25) (layer B.Cu) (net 2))
 (segment (start 35.56 -5.08) (end 35.56 -7.62) (width 0.25) (layer B.Cu) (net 2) (status 20))
 (segment (start 30.48 2.54) (end 30.48 -2.54) (width 0.25) (layer B.Cu) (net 9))
 (segment (start 27.94 -2.54) (end 20.32 -2.54) (width 0.25) (layer B.Cu) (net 9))
 (segment (start 20.32 -2.54) (end 20.32 -5.08) (width 0.25) (layer B.Cu) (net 9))
 (segment (start 27.94 -2.54) (end 30.48 -2.54) (width 0.25) (layer B.Cu) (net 9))
 (segment (start 12.7 -5.08) (end 20.32 -5.08) (width 0.25) (layer B.Cu) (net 9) (status 10))
 (segment (start 30.48 -5.08) (end 30.48 -12.7) (width 0.25) (layer B.Cu) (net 11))
 (segment (start 10.16 -12.7) (end 10.16 -10.16) (width 0.25) (layer B.Cu) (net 11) (status 20))
 (segment (start 30.48 -12.7) (end 10.16 -12.7) (width 0.25) (layer B.Cu) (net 11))
 (segment (start 35.56 2.54) (end 35.56 5.08) (width 0.25) (layer B.Cu) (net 12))
 (segment (start 12.7 0) (end 15.24 0) (width 0.25) (layer B.Cu) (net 12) (status 10))
 (segment (start 15.24 5.08) (end 35.56 5.08) (width 0.25) (layer B.Cu) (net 12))
 (segment (start 15.24 0) (end 15.24 5.08) (width 0.25) (layer B.Cu) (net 12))
 (segment (start 27.94 -5.08) (end 27.94 -10.16) (width 0.25) (layer B.Cu) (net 13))
 (segment (start 12.7 -10.16) (end 27.94 -10.16) (width 0.25) (layer B.Cu) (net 13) (status 10))
 (segment (start 38.1 3.81) (end 38.1 2.54) (width 0.25) (layer F.Cu) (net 14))
 (segment (start 10.16 0) (end 11.43 -1.27) (width 0.25) (layer F.Cu) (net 14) (status 10))
 (segment (start 16.51 3.81) (end 38.1 3.81) (width 0.25) (layer F.Cu) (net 14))
 (segment (start 16.51 -1.27) (end 16.51 3.81) (width 0.25) (layer F.Cu) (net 14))
 (segment (start 11.43 -1.27) (end 16.51 -1.27) (width 0.25) (layer F.Cu) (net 14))
 (segment (start 25.4 -5.08) (end 25.4 -8.89) (width 0.25) (layer B.Cu) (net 15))
 (segment (start 10.16 -7.62) (end 11.43 -8.89) (width 0.25) (layer B.Cu) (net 15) (status 10))
 (segment (start 11.43 -8.89) (end 25.4 -8.89) (width 0.25) (layer B.Cu) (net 15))
 (segment (start 40.64 2.54) (end 40.64 6.35) (width 0.25) (layer F.Cu) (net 16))
 (segment (start 10.16 2.54) (end 11.43 1.27) (width 0.25) (layer F.Cu) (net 16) (status 10))
 (segment (start 13.97 6.35) (end 40.64 6.35) (width 0.25) (layer F.Cu) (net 16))
 (segment (start 13.97 1.27) (end 13.97 6.35) (width 0.25) (layer F.Cu) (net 16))
 (segment (start 11.43 1.27) (end 13.97 1.27) (width 0.25) (layer F.Cu) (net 16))
 (segment (start 22.86 -5.08) (end 22.86 -7.62) (width 0.25) (layer B.Cu) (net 17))
 (segment (start 12.7 -7.62) (end 22.86 -7.62) (width 0.25) (layer B.Cu) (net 17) (status 10))
 (segment (start 12.7 2.54) (end 11.43 3.81) (width 0.25) (layer B.Cu) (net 19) (status 10))
 (segment (start 5.04 3.77) (end 5.04 -5.04) (width 0.25) (layer B.Cu) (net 19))
 (segment (start 5.08 3.81) (end 5.04 3.77) (width 0.25) (layer B.Cu) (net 19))
 (segment (start 11.43 3.81) (end 5.08 3.81) (width 0.25) (layer B.Cu) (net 19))
 (segment (start 88.9 -7.62) (end 91.44 -7.62) (width 0.25) (layer B.Cu) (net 20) (status 20))
 (segment (start 91.44 -7.62) (end 91.44 -5.08) (width 0.25) (layer B.Cu) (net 20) (status 30))
 (segment (start 86.36 -5.08) (end 86.36 -2.54) (width 0.25) (layer B.Cu) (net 21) (status 10))
 (segment (start 86.36 -2.54) (end 88.9 -2.54) (width 0.25) (layer B.Cu) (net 21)))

